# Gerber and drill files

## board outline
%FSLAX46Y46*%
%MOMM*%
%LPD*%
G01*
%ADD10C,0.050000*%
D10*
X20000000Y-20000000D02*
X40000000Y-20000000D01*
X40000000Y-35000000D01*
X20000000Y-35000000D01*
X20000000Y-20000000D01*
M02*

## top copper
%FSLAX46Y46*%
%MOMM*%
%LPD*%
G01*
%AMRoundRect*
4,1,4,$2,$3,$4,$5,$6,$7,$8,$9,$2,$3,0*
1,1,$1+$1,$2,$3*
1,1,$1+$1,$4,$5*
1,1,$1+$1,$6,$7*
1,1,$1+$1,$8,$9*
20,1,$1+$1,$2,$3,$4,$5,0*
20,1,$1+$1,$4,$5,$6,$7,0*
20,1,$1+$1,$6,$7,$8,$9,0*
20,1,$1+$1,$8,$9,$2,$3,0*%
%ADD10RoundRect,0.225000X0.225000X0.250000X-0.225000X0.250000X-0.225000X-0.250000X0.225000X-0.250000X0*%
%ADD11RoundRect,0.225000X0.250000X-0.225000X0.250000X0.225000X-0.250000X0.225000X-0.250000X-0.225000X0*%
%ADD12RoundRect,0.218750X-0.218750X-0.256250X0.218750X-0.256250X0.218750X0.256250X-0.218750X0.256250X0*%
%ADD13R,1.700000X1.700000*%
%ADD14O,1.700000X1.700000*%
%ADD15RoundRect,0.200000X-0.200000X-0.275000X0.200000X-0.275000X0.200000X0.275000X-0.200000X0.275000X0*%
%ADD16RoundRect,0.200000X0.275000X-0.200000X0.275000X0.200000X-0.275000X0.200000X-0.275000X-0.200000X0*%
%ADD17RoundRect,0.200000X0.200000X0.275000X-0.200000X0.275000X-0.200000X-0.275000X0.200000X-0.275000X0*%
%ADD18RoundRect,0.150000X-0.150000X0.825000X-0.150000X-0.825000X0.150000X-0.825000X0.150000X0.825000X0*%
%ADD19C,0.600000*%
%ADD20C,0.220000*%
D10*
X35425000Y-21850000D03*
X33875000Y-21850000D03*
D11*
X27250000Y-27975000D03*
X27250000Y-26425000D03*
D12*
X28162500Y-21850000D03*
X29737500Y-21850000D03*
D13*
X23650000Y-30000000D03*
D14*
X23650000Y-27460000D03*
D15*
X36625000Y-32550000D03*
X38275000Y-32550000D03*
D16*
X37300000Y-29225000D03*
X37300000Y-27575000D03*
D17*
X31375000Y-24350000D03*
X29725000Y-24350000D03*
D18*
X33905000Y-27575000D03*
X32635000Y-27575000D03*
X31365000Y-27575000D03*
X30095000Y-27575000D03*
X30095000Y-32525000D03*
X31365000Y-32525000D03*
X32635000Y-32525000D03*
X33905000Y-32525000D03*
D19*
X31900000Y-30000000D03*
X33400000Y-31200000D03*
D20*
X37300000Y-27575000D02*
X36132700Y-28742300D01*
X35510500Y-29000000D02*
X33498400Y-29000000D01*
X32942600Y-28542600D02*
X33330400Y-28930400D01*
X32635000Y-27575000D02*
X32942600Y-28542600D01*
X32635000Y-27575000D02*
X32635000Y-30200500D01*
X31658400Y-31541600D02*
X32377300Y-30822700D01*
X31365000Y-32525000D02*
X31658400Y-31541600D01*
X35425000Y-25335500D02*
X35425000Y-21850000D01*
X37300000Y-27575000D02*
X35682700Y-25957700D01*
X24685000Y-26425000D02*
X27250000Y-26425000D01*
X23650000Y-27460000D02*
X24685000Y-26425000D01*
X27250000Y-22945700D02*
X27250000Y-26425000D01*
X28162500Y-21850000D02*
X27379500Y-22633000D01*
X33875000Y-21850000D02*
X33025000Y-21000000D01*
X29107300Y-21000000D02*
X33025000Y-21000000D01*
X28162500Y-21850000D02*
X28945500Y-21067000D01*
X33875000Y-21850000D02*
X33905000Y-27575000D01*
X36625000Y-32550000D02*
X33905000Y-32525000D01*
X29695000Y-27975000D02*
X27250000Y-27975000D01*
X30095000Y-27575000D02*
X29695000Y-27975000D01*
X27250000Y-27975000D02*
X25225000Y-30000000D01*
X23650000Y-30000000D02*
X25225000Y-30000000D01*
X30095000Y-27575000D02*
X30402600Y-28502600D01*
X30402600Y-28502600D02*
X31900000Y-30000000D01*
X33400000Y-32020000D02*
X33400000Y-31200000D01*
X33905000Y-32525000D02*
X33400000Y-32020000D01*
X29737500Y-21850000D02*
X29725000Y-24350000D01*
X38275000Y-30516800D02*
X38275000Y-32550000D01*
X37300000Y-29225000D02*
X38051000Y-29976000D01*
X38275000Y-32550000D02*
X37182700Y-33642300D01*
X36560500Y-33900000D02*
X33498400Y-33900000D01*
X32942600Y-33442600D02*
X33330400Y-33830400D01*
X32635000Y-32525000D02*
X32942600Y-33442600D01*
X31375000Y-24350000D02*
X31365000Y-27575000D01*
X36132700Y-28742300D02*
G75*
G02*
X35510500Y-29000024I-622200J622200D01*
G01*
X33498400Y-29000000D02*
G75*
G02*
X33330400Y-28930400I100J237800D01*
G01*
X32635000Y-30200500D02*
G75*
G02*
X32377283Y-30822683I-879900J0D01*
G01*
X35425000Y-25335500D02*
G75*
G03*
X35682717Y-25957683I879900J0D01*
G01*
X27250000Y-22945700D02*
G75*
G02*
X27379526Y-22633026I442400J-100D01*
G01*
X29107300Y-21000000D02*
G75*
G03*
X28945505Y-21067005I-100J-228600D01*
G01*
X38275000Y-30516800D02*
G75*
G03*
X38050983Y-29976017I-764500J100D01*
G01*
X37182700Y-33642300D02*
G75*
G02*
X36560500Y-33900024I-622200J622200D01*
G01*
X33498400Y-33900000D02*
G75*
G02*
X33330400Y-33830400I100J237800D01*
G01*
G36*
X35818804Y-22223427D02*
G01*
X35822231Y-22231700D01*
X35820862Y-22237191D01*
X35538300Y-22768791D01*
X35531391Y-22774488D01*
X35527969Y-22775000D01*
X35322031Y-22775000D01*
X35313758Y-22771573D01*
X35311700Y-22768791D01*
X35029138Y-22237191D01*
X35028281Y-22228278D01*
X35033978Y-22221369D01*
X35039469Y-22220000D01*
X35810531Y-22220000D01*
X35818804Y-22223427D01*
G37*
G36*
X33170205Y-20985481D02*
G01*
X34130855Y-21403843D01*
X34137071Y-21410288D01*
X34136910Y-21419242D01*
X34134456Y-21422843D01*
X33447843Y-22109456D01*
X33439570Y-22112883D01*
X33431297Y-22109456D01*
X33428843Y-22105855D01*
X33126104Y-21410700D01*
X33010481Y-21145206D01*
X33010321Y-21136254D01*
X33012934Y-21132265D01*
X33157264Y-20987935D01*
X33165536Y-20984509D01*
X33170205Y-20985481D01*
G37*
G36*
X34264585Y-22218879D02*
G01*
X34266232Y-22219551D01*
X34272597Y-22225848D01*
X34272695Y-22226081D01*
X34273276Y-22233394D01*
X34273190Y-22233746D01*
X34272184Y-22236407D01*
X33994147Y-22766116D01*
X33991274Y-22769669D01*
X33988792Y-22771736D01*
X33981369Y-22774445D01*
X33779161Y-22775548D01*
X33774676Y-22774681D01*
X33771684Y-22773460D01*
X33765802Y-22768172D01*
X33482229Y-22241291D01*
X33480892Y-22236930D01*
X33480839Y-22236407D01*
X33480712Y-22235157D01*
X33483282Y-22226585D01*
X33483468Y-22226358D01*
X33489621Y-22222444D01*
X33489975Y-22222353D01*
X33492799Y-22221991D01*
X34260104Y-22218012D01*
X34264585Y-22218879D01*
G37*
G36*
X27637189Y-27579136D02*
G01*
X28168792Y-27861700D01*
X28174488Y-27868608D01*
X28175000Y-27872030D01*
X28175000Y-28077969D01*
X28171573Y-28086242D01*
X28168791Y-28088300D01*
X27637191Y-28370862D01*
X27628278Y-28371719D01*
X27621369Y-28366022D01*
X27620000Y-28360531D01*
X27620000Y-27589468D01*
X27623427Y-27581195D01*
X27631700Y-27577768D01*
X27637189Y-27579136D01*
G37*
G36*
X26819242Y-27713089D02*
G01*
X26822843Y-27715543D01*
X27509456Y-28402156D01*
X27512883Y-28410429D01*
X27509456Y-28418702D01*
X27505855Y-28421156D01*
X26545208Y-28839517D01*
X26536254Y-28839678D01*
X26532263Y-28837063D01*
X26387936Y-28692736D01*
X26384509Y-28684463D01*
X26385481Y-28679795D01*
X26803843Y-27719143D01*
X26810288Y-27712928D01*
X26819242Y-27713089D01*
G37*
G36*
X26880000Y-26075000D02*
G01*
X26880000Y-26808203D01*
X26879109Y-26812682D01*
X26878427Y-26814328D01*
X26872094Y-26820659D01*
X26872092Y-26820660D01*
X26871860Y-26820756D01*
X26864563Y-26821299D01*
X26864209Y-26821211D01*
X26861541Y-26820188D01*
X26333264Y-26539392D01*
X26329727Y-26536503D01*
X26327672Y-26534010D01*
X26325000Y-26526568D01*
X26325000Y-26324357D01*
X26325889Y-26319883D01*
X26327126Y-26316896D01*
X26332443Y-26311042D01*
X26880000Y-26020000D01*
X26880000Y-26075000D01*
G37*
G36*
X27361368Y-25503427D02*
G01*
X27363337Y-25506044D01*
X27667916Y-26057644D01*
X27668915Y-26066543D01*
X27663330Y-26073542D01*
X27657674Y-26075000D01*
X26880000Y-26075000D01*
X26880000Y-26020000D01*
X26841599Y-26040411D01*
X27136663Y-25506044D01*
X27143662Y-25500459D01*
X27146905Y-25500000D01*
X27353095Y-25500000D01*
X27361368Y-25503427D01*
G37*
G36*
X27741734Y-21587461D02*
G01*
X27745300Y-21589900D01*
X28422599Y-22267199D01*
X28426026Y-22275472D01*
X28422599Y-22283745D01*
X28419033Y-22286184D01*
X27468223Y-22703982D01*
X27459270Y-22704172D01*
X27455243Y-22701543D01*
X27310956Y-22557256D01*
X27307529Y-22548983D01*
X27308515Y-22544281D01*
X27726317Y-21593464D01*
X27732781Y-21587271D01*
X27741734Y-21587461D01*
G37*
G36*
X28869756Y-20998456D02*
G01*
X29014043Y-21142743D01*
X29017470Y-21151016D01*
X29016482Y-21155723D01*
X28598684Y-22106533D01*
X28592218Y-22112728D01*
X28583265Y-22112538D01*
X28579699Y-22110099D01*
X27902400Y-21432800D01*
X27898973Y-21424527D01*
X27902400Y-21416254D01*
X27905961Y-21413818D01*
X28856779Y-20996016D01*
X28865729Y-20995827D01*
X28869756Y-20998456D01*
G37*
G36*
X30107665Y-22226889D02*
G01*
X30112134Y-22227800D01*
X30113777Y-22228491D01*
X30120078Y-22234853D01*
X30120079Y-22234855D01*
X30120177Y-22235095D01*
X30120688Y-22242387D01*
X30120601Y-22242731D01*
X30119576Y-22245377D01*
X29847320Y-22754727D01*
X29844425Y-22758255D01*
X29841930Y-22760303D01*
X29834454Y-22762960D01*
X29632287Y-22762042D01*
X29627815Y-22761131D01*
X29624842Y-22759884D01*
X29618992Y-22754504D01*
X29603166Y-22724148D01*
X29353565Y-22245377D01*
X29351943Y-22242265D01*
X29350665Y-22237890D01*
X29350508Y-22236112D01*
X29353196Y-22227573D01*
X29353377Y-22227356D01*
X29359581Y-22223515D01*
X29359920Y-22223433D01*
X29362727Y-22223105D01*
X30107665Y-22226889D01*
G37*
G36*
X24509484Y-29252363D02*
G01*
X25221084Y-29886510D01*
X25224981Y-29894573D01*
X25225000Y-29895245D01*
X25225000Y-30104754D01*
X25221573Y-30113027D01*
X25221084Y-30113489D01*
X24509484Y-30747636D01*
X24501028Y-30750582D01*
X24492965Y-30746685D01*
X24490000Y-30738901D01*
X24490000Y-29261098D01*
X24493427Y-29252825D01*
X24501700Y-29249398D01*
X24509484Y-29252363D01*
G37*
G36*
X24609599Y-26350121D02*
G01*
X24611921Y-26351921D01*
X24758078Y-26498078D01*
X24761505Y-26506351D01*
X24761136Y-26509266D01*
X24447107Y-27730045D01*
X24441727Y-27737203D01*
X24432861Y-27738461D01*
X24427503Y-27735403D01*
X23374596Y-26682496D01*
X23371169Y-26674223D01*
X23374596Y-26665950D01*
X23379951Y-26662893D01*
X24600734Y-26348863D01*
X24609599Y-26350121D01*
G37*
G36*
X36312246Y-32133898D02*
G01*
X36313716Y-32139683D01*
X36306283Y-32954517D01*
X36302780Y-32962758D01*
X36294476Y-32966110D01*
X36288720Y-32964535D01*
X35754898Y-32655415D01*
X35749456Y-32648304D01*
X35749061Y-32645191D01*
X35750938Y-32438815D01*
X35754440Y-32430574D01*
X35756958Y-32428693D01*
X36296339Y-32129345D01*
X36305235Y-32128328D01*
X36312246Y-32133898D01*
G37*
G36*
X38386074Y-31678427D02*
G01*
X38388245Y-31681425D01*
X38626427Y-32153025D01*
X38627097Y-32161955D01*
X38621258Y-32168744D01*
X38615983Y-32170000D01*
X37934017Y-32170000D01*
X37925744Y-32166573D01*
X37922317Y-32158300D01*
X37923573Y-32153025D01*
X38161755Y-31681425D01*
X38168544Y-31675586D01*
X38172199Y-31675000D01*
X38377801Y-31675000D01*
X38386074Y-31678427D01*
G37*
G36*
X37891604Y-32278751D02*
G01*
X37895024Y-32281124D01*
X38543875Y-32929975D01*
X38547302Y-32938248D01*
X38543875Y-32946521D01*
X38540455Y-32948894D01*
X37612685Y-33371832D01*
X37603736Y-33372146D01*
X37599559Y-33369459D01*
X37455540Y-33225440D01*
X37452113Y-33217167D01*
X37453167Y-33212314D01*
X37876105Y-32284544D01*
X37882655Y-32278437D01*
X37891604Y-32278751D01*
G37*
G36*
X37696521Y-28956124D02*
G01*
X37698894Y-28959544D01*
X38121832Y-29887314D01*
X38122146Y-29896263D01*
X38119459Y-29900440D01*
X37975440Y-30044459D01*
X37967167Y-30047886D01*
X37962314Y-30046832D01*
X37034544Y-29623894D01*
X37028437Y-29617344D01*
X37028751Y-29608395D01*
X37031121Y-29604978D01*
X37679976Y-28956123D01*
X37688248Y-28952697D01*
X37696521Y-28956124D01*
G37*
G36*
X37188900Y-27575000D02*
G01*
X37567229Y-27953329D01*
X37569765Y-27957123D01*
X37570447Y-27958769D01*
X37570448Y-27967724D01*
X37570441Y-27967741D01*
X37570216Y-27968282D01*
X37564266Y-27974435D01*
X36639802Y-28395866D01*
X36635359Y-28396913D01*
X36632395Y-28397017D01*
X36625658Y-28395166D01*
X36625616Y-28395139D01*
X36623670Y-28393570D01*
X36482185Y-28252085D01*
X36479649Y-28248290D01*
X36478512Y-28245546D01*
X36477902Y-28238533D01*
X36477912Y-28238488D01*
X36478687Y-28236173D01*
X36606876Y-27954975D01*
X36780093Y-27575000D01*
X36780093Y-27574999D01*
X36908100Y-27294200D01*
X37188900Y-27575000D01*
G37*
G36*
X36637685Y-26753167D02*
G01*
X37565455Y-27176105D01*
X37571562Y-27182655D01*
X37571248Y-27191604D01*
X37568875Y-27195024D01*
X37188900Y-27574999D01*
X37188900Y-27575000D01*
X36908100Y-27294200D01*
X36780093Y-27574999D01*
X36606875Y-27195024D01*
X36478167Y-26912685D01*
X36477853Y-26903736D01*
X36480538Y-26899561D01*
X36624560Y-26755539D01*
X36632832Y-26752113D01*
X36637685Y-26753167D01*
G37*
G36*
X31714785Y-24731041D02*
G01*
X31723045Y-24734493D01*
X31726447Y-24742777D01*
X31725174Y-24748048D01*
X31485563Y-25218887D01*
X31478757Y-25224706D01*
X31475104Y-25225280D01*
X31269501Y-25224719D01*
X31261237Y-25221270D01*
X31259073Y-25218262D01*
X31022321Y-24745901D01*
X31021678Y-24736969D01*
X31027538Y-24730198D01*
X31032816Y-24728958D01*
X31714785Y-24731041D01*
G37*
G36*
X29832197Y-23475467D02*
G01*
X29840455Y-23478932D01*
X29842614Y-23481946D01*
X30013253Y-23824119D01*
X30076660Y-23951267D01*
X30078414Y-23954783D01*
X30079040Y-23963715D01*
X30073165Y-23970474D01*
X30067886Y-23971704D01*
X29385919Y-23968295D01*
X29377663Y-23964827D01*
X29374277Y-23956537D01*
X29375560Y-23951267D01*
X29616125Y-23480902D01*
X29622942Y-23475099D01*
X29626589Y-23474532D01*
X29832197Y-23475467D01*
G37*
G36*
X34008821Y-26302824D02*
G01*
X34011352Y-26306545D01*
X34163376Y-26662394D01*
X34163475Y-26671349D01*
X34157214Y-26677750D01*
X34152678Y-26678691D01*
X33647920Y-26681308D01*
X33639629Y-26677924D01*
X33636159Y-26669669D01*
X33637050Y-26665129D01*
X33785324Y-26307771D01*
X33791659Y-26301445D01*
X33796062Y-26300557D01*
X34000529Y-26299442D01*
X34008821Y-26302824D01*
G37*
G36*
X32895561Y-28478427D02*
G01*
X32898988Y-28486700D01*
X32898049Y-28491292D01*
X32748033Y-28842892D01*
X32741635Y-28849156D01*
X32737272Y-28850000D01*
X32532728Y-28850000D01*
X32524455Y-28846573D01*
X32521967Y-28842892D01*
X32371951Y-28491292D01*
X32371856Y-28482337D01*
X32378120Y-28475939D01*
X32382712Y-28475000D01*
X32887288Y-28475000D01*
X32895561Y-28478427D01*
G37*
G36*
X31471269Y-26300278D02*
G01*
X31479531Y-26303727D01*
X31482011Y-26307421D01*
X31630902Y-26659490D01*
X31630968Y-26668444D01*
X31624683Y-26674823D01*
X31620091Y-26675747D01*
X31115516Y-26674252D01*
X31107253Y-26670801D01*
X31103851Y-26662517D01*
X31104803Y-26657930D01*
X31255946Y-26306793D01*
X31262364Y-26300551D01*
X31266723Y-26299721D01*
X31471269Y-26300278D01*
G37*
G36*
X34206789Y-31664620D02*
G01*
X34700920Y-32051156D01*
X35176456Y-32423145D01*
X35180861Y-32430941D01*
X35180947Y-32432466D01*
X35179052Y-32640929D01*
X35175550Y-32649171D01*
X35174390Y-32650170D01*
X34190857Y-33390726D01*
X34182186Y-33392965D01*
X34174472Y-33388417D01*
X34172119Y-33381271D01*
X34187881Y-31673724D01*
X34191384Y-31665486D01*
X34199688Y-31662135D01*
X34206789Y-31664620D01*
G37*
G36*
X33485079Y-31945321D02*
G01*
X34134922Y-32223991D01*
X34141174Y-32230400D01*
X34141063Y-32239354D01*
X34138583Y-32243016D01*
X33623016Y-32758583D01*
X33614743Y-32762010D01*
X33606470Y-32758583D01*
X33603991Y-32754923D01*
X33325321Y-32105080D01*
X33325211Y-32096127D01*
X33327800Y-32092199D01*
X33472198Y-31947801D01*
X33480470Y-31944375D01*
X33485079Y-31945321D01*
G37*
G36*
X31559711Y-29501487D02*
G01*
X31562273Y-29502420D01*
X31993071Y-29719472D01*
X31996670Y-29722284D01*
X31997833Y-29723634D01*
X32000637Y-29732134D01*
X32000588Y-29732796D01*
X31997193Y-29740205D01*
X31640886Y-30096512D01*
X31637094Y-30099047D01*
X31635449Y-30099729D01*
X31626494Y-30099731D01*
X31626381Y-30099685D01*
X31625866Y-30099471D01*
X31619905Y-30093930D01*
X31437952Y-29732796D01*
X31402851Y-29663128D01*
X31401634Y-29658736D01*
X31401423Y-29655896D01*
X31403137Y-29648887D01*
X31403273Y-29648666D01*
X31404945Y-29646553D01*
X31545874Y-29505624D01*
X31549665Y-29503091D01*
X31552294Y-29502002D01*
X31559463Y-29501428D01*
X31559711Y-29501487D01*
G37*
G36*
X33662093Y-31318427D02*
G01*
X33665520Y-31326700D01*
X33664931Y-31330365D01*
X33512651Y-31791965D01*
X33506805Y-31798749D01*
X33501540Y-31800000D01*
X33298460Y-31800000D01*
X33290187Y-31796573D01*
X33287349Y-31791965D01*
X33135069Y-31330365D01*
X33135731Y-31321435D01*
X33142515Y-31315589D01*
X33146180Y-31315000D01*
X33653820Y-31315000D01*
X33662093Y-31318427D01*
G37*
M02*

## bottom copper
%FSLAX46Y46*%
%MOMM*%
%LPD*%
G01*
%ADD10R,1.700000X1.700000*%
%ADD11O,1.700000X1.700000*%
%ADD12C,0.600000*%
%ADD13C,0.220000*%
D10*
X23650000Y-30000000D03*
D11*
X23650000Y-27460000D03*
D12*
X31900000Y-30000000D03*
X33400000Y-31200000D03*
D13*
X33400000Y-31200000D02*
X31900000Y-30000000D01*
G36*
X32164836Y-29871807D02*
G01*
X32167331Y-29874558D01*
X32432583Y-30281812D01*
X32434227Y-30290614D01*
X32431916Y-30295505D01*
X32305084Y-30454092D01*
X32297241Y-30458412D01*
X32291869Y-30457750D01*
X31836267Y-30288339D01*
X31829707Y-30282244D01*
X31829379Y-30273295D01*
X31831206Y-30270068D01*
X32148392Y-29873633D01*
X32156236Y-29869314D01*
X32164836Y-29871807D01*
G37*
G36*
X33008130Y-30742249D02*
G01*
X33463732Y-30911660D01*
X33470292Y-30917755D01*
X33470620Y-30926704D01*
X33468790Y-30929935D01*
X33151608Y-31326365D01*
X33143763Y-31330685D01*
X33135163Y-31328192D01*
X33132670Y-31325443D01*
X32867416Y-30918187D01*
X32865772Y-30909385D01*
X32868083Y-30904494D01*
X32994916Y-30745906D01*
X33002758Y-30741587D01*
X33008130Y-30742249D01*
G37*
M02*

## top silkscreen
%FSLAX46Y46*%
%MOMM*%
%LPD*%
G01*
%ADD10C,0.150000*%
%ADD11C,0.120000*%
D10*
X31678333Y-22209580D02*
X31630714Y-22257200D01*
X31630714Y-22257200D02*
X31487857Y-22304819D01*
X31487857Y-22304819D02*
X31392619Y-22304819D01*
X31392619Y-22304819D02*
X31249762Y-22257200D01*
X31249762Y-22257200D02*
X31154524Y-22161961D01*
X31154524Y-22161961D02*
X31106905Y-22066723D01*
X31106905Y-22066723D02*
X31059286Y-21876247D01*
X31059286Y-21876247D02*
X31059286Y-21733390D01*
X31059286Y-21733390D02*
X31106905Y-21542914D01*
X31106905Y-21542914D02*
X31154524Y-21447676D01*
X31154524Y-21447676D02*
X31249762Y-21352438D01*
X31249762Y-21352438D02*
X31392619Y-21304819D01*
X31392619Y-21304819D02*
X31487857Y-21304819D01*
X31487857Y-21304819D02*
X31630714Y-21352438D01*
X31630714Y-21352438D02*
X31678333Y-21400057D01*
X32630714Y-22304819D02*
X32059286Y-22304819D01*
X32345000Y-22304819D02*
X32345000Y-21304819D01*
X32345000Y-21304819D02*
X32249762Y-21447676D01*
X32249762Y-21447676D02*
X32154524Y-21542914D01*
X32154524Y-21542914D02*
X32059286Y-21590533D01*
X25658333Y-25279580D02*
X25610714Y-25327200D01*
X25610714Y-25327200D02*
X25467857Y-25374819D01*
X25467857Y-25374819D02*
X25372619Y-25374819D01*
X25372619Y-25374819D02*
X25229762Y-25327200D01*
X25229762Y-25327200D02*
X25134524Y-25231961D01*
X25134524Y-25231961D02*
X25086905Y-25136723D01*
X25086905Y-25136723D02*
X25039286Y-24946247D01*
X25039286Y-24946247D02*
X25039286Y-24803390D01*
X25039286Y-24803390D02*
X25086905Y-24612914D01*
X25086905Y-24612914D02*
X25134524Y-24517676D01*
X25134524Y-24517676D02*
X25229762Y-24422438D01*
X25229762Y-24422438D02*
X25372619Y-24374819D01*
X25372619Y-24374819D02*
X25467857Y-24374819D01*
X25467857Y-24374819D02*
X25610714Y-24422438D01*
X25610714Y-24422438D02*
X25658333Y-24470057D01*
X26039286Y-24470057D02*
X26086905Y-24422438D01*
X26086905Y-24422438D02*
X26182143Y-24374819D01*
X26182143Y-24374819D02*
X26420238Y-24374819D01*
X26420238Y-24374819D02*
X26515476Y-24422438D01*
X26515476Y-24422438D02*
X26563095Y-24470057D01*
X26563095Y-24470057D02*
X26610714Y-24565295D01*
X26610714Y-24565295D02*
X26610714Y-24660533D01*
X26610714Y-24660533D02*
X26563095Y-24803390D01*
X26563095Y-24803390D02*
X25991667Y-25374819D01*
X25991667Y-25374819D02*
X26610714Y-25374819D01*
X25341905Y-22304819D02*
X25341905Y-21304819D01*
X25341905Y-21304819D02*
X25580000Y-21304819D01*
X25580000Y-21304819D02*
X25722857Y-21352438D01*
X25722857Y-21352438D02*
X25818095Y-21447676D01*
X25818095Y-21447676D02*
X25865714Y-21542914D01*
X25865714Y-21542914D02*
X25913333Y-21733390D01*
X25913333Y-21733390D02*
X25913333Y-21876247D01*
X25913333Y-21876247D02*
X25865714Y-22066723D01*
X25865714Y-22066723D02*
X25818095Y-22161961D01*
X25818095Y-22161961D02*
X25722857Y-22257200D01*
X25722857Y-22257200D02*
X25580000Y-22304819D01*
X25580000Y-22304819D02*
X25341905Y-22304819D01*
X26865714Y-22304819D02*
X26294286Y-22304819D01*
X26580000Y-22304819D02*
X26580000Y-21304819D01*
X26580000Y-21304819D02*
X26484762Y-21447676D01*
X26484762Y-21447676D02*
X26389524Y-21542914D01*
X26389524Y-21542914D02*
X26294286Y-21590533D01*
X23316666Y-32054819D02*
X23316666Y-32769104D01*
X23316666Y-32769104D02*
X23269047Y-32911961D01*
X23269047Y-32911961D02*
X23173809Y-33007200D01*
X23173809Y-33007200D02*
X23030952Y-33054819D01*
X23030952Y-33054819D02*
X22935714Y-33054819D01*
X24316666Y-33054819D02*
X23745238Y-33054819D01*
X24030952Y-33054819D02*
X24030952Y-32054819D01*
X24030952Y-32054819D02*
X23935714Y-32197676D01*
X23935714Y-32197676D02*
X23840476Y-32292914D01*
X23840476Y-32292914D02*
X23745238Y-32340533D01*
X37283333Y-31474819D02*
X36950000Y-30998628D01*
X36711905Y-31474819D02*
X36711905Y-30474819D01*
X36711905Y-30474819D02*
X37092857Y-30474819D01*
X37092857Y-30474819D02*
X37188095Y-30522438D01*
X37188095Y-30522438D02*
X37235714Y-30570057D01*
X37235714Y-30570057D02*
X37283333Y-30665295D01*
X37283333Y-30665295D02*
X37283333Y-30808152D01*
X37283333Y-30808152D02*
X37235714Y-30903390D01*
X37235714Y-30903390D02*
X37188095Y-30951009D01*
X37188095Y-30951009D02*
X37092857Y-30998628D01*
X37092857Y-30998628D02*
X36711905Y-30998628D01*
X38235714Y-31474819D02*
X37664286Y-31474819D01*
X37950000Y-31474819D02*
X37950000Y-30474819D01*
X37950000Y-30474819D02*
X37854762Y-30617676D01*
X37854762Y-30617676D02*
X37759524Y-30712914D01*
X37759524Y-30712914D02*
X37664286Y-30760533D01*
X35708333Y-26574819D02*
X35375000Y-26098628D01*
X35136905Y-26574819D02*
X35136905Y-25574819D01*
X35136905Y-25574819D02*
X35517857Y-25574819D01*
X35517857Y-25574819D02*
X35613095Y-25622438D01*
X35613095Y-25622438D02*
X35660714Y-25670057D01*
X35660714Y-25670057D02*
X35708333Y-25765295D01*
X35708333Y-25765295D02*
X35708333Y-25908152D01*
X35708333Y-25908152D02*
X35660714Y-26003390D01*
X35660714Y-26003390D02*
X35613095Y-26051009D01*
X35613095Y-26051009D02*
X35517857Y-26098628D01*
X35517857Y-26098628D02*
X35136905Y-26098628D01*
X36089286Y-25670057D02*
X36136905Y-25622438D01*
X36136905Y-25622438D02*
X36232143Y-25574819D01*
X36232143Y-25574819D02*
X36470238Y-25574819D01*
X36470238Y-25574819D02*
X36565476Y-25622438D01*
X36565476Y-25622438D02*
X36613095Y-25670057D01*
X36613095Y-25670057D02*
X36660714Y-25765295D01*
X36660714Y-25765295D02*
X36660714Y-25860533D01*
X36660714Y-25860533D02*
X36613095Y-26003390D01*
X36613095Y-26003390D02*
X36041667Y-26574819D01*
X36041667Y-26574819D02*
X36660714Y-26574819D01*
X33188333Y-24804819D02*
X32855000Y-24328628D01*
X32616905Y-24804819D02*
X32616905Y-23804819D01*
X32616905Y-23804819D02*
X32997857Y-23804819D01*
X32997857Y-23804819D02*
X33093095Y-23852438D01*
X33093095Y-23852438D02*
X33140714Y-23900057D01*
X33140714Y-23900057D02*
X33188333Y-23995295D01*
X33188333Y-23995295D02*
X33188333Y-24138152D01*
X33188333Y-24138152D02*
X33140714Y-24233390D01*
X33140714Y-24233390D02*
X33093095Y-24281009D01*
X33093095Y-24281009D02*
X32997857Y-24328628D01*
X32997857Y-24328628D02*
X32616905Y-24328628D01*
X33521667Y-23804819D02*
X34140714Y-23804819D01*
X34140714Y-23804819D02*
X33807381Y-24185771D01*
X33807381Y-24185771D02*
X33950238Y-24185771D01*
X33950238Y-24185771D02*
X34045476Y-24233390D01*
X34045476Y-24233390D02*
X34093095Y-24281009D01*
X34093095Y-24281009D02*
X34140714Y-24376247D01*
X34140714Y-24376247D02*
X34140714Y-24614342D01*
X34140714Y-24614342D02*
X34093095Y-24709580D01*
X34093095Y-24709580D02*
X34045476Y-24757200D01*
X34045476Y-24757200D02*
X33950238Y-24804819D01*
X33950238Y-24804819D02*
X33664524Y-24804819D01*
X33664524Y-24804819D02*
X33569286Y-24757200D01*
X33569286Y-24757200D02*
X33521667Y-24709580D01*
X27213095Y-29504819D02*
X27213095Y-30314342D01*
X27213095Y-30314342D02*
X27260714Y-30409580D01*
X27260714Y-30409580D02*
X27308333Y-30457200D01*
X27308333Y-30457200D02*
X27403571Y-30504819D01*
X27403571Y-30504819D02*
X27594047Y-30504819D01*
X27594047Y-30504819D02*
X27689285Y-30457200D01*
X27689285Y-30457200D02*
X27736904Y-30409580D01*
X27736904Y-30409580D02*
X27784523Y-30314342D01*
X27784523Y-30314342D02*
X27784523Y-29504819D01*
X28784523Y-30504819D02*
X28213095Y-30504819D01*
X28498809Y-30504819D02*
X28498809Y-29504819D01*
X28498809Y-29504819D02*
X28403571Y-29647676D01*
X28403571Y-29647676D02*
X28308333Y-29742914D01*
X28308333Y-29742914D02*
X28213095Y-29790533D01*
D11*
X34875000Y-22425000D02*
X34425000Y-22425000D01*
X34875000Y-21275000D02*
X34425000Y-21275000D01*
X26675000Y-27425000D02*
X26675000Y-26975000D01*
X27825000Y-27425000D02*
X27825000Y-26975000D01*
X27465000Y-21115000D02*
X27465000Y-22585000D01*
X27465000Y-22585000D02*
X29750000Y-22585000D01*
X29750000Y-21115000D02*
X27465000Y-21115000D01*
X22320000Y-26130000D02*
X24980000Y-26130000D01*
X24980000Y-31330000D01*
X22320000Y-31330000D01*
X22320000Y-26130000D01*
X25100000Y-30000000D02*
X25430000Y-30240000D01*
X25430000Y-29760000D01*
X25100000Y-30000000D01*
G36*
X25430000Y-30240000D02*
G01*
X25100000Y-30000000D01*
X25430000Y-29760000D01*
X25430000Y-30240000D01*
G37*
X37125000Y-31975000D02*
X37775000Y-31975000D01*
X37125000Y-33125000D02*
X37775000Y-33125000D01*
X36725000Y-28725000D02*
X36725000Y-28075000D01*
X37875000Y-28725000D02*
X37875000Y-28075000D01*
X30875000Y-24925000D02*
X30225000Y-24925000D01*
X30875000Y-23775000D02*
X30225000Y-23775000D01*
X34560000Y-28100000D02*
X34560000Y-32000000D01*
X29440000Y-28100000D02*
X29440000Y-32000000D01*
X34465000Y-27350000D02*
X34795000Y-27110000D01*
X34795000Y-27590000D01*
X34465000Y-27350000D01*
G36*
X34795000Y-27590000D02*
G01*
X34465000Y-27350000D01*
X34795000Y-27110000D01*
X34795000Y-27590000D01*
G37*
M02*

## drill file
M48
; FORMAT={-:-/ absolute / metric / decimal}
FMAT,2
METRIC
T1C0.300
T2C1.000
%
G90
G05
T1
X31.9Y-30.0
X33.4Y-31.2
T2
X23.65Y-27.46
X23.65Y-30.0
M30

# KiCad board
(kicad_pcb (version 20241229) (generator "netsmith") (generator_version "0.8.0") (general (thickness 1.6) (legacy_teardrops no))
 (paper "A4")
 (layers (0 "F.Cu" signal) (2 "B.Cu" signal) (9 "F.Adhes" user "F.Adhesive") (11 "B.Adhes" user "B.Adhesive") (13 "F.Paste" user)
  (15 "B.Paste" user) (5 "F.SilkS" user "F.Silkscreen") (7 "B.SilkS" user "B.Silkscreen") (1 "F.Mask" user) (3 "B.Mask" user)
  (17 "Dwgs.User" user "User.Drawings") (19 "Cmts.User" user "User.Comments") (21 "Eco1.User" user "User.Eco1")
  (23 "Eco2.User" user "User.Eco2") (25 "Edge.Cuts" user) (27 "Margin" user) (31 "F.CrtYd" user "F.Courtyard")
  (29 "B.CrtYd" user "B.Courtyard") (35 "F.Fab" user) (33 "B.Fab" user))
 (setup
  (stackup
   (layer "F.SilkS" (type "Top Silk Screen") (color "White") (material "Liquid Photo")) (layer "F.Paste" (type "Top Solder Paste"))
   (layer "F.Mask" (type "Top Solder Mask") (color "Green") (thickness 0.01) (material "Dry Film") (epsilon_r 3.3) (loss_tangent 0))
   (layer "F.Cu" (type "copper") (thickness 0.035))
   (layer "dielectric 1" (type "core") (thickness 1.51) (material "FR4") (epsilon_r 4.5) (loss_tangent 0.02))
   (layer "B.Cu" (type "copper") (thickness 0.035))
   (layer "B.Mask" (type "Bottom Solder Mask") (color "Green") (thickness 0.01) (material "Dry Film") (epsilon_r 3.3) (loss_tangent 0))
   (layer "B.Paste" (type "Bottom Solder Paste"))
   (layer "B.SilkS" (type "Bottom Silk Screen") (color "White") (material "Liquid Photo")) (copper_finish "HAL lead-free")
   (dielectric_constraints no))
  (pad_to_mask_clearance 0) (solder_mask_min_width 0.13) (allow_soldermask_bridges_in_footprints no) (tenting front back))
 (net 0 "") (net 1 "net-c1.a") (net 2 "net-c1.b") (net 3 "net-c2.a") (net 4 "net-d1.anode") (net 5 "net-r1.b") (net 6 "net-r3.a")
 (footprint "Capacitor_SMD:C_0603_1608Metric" (layer "F.Cu") (at 34.65 21.85 180)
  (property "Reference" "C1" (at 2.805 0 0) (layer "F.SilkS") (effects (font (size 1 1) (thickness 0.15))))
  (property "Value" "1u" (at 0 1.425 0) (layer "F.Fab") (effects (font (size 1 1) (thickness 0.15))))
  (pad "1" smd roundrect (at -0.775 0 180) (size 0.9 0.95) (layers "F.Cu" "F.Mask" "F.Paste") (roundrect_rratio 0.25) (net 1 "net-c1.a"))
  (pad "2" smd roundrect (at 0.775 0 180) (size 0.9 0.95) (layers "F.Cu" "F.Mask" "F.Paste") (roundrect_rratio 0.25) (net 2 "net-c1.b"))
  (fp_line (start -0.225 -0.575) (end 0.225 -0.575) (stroke (width 0.12) (type solid)) (layer "F.SilkS"))
  (fp_line (start -0.225 0.575) (end 0.225 0.575) (stroke (width 0.12) (type solid)) (layer "F.SilkS")))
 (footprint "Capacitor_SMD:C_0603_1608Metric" (layer "F.Cu") (at 27.25 27.2 90)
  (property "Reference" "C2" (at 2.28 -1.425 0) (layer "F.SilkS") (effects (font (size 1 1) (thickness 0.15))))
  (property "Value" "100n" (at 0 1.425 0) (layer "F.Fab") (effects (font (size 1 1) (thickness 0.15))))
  (pad "1" smd roundrect (at -0.775 0 90) (size 0.9 0.95) (layers "F.Cu" "F.Mask" "F.Paste") (roundrect_rratio 0.25) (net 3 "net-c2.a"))
  (pad "2" smd roundrect (at 0.775 0 90) (size 0.9 0.95) (layers "F.Cu" "F.Mask" "F.Paste") (roundrect_rratio 0.25) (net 2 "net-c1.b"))
  (fp_line (start -0.225 -0.575) (end 0.225 -0.575) (stroke (width 0.12) (type solid)) (layer "F.SilkS"))
  (fp_line (start -0.225 0.575) (end 0.225 0.575) (stroke (width 0.12) (type solid)) (layer "F.SilkS")))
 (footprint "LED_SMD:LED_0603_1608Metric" (layer "F.Cu") (at 28.95 21.85)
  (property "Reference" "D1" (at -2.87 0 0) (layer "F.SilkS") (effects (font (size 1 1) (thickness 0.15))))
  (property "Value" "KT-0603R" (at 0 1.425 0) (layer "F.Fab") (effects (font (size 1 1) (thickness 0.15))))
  (pad "1" smd roundrect (at -0.7875 0) (size 0.875 0.95) (layers "F.Cu" "F.Mask" "F.Paste") (roundrect_rratio 0.25) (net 2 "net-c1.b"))
  (pad "2" smd roundrect (at 0.7875 0) (size 0.875 0.95) (layers "F.Cu" "F.Mask" "F.Paste") (roundrect_rratio 0.25) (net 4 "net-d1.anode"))
  (fp_line (start -1.485 -0.735) (end -1.485 0.735) (stroke (width 0.12) (type solid)) (layer "F.SilkS"))
  (fp_line (start -1.485 0.735) (end 0.8 0.735) (stroke (width 0.12) (type solid)) (layer "F.SilkS"))
  (fp_line (start 0.8 -0.735) (end -1.485 -0.735) (stroke (width 0.12) (type solid)) (layer "F.SilkS")))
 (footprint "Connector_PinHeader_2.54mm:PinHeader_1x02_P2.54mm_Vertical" (layer "F.Cu") (at 23.65 30 180)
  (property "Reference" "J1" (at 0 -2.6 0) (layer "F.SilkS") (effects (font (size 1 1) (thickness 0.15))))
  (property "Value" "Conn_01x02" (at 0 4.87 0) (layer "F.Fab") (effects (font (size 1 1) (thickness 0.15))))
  (pad "1" thru_hole rect (at 0 0 180) (size 1.7 1.7) (drill 1) (layers "*.Cu" "*.Mask") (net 3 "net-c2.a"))
  (pad "2" thru_hole oval (at 0 2.54 180) (size 1.7 1.7) (drill 1) (layers "*.Cu" "*.Mask") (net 2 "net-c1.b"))
  (fp_rect (start -1.33 -1.33) (end 1.33 3.87) (stroke (width 0.12) (type solid)) (fill no) (layer "F.SilkS"))
  (fp_poly (pts (xy -1.45 0) (xy -1.78 -0.24) (xy -1.78 0.24)) (stroke (width 0.12) (type solid)) (fill solid) (layer "F.SilkS")))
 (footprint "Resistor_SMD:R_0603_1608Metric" (layer "F.Cu") (at 37.45 32.55)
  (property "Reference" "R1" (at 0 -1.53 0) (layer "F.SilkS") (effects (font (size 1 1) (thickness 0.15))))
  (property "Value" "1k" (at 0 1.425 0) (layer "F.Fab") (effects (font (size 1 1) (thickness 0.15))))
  (pad "1" smd roundrect (at -0.825 0) (size 0.8 0.95) (layers "F.Cu" "F.Mask" "F.Paste") (roundrect_rratio 0.25) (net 3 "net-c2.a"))
  (pad "2" smd roundrect (at 0.825 0) (size 0.8 0.95) (layers "F.Cu" "F.Mask" "F.Paste") (roundrect_rratio 0.25) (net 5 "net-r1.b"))
  (fp_line (start -0.325 -0.575) (end 0.325 -0.575) (stroke (width 0.12) (type solid)) (layer "F.SilkS"))
  (fp_line (start -0.325 0.575) (end 0.325 0.575) (stroke (width 0.12) (type solid)) (layer "F.SilkS")))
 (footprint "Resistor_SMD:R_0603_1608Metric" (layer "F.Cu") (at 37.3 28.4 90)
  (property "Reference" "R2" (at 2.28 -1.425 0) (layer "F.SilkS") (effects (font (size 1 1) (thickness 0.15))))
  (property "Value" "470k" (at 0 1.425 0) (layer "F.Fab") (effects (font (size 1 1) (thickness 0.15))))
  (pad "1" smd roundrect (at -0.825 0 90) (size 0.8 0.95) (layers "F.Cu" "F.Mask" "F.Paste") (roundrect_rratio 0.25) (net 5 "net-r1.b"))
  (pad "2" smd roundrect (at 0.825 0 90) (size 0.8 0.95) (layers "F.Cu" "F.Mask" "F.Paste") (roundrect_rratio 0.25) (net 1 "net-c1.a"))
  (fp_line (start -0.325 -0.575) (end 0.325 -0.575) (stroke (width 0.12) (type solid)) (layer "F.SilkS"))
  (fp_line (start -0.325 0.575) (end 0.325 0.575) (stroke (width 0.12) (type solid)) (layer "F.SilkS")))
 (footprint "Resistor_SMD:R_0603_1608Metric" (layer "F.Cu") (at 30.55 24.35 180)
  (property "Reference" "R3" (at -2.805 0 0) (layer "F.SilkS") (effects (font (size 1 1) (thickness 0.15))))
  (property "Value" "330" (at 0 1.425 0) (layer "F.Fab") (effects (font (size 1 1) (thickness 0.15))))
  (pad "1" smd roundrect (at -0.825 0 180) (size 0.8 0.95) (layers "F.Cu" "F.Mask" "F.Paste") (roundrect_rratio 0.25) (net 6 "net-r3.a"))
  (pad "2" smd roundrect (at 0.825 0 180) (size 0.8 0.95) (layers "F.Cu" "F.Mask" "F.Paste") (roundrect_rratio 0.25) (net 4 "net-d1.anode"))
  (fp_line (start -0.325 -0.575) (end 0.325 -0.575) (stroke (width 0.12) (type solid)) (layer "F.SilkS"))
  (fp_line (start -0.325 0.575) (end 0.325 0.575) (stroke (width 0.12) (type solid)) (layer "F.SilkS")))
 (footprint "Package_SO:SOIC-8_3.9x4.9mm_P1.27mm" (layer "F.Cu") (at 32 30.05 270)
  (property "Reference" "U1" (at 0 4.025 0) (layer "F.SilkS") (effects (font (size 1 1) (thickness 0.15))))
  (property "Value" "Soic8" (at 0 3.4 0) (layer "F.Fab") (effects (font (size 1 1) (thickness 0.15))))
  (pad "1" smd roundrect (at -2.475 -1.905 270) (size 1.95 0.6) (layers "F.Cu" "F.Mask" "F.Paste") (roundrect_rratio 0.25)
   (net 2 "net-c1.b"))
  (pad "2" smd roundrect (at -2.475 -0.635 270) (size 1.95 0.6) (layers "F.Cu" "F.Mask" "F.Paste") (roundrect_rratio 0.25)
   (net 1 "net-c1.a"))
  (pad "3" smd roundrect (at -2.475 0.635 270) (size 1.95 0.6) (layers "F.Cu" "F.Mask" "F.Paste") (roundrect_rratio 0.25) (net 6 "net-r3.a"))
  (pad "4" smd roundrect (at -2.475 1.905 270) (size 1.95 0.6) (layers "F.Cu" "F.Mask" "F.Paste") (roundrect_rratio 0.25) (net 3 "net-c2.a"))
  (pad "5" smd roundrect (at 2.475 1.905 270) (size 1.95 0.6) (layers "F.Cu" "F.Mask" "F.Paste") (roundrect_rratio 0.25))
  (pad "6" smd roundrect (at 2.475 0.635 270) (size 1.95 0.6) (layers "F.Cu" "F.Mask" "F.Paste") (roundrect_rratio 0.25) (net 1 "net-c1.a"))
  (pad "7" smd roundrect (at 2.475 -0.635 270) (size 1.95 0.6) (layers "F.Cu" "F.Mask" "F.Paste") (roundrect_rratio 0.25) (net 5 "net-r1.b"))
  (pad "8" smd roundrect (at 2.475 -1.905 270) (size 1.95 0.6) (layers "F.Cu" "F.Mask" "F.Paste") (roundrect_rratio 0.25) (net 3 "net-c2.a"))
  (fp_line (start -1.95 -2.56) (end 1.95 -2.56) (stroke (width 0.12) (type solid)) (layer "F.SilkS"))
  (fp_line (start -1.95 2.56) (end 1.95 2.56) (stroke (width 0.12) (type solid)) (layer "F.SilkS"))
  (fp_poly (pts (xy -2.7 -2.465) (xy -2.94 -2.795) (xy -2.46 -2.795)) (stroke (width 0.12) (type solid)) (fill solid) (layer "F.SilkS")))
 (segment (start 37.3 27.575) (end 36.1327 28.7423) (width 0.22) (layer "F.Cu") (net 1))
 (segment (start 35.5105 29) (end 33.4984 29) (width 0.22) (layer "F.Cu") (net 1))
 (segment (start 32.9426 28.5426) (end 33.3304 28.9304) (width 0.22) (layer "F.Cu") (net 1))
 (segment (start 32.635 27.575) (end 32.9426 28.5426) (width 0.22) (layer "F.Cu") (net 1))
 (segment (start 32.635 27.575) (end 32.635 30.2005) (width 0.22) (layer "F.Cu") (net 1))
 (segment (start 31.6584 31.5416) (end 32.3773 30.8227) (width 0.22) (layer "F.Cu") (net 1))
 (segment (start 31.365 32.525) (end 31.6584 31.5416) (width 0.22) (layer "F.Cu") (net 1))
 (segment (start 35.425 25.3355) (end 35.425 21.85) (width 0.22) (layer "F.Cu") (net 1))
 (segment (start 37.3 27.575) (end 35.6827 25.9577) (width 0.22) (layer "F.Cu") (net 1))
 (segment (start 24.685 26.425) (end 27.25 26.425) (width 0.22) (layer "F.Cu") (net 2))
 (segment (start 23.65 27.46) (end 24.685 26.425) (width 0.22) (layer "F.Cu") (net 2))
 (segment (start 27.25 22.9457) (end 27.25 26.425) (width 0.22) (layer "F.Cu") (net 2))
 (segment (start 28.1625 21.85) (end 27.3795 22.633) (width 0.22) (layer "F.Cu") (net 2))
 (segment (start 33.875 21.85) (end 33.025 21) (width 0.22) (layer "F.Cu") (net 2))
 (segment (start 29.1073 21) (end 33.025 21) (width 0.22) (layer "F.Cu") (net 2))
 (segment (start 28.1625 21.85) (end 28.9455 21.067) (width 0.22) (layer "F.Cu") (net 2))
 (segment (start 33.875 21.85) (end 33.905 27.575) (width 0.22) (layer "F.Cu") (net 2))
 (segment (start 36.625 32.55) (end 33.905 32.525) (width 0.22) (layer "F.Cu") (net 3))
 (segment (start 29.695 27.975) (end 27.25 27.975) (width 0.22) (layer "F.Cu") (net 3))
 (segment (start 30.095 27.575) (end 29.695 27.975) (width 0.22) (layer "F.Cu") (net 3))
 (segment (start 27.25 27.975) (end 25.225 30) (width 0.22) (layer "F.Cu") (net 3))
 (segment (start 23.65 30) (end 25.225 30) (width 0.22) (layer "F.Cu") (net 3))
 (segment (start 30.095 27.575) (end 30.4026 28.5026) (width 0.22) (layer "F.Cu") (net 3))
 (segment (start 30.4026 28.5026) (end 31.9 30) (width 0.22) (layer "F.Cu") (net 3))
 (segment (start 33.4 31.2) (end 31.9 30) (width 0.22) (layer "B.Cu") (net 3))
 (segment (start 33.4 32.02) (end 33.4 31.2) (width 0.22) (layer "F.Cu") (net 3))
 (segment (start 33.905 32.525) (end 33.4 32.02) (width 0.22) (layer "F.Cu") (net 3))
 (segment (start 29.7375 21.85) (end 29.725 24.35) (width 0.22) (layer "F.Cu") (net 4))
 (segment (start 38.275 30.5168) (end 38.275 32.55) (width 0.22) (layer "F.Cu") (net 5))
 (segment (start 37.3 29.225) (end 38.051 29.976) (width 0.22) (layer "F.Cu") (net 5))
 (segment (start 38.275 32.55) (end 37.1827 33.6423) (width 0.22) (layer "F.Cu") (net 5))
 (segment (start 36.5605 33.9) (end 33.4984 33.9) (width 0.22) (layer "F.Cu") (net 5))
 (segment (start 32.9426 33.4426) (end 33.3304 33.8304) (width 0.22) (layer "F.Cu") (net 5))
 (segment (start 32.635 32.525) (end 32.9426 33.4426) (width 0.22) (layer "F.Cu") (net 5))
 (segment (start 31.375 24.35) (end 31.365 27.575) (width 0.22) (layer "F.Cu") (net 6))
 (arc (start 36.1327 28.7423) (mid 35.8473 28.933) (end 35.5105 29) (width 0.22) (layer "F.Cu") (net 1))
 (arc (start 33.4984 29) (mid 33.4075 28.9819) (end 33.3304 28.9304) (width 0.22) (layer "F.Cu") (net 1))
 (arc (start 32.635 30.2005) (mid 32.568 30.5373) (end 32.3773 30.8227) (width 0.22) (layer "F.Cu") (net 1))
 (arc (start 35.425 25.3355) (mid 35.492 25.6723) (end 35.6827 25.9577) (width 0.22) (layer "F.Cu") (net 1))
 (arc (start 27.25 22.9457) (mid 27.2837 22.7764) (end 27.3795 22.633) (width 0.22) (layer "F.Cu") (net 2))
 (arc (start 29.1073 21) (mid 29.0197 21.0174) (end 28.9455 21.067) (width 0.22) (layer "F.Cu") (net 2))
 (arc (start 38.275 30.5168) (mid 38.2168 30.2241) (end 38.051 29.976) (width 0.22) (layer "F.Cu") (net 5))
 (arc (start 37.1827 33.6423) (mid 36.8973 33.833) (end 36.5605 33.9) (width 0.22) (layer "F.Cu") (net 5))
 (arc (start 33.4984 33.9) (mid 33.4075 33.8819) (end 33.3304 33.8304) (width 0.22) (layer "F.Cu") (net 5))
 (via (at 31.9 30) (size 0.6) (drill 0.3) (layers "F.Cu" "B.Cu") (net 3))
 (via (at 33.4 31.2) (size 0.6) (drill 0.3) (layers "F.Cu" "B.Cu") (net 3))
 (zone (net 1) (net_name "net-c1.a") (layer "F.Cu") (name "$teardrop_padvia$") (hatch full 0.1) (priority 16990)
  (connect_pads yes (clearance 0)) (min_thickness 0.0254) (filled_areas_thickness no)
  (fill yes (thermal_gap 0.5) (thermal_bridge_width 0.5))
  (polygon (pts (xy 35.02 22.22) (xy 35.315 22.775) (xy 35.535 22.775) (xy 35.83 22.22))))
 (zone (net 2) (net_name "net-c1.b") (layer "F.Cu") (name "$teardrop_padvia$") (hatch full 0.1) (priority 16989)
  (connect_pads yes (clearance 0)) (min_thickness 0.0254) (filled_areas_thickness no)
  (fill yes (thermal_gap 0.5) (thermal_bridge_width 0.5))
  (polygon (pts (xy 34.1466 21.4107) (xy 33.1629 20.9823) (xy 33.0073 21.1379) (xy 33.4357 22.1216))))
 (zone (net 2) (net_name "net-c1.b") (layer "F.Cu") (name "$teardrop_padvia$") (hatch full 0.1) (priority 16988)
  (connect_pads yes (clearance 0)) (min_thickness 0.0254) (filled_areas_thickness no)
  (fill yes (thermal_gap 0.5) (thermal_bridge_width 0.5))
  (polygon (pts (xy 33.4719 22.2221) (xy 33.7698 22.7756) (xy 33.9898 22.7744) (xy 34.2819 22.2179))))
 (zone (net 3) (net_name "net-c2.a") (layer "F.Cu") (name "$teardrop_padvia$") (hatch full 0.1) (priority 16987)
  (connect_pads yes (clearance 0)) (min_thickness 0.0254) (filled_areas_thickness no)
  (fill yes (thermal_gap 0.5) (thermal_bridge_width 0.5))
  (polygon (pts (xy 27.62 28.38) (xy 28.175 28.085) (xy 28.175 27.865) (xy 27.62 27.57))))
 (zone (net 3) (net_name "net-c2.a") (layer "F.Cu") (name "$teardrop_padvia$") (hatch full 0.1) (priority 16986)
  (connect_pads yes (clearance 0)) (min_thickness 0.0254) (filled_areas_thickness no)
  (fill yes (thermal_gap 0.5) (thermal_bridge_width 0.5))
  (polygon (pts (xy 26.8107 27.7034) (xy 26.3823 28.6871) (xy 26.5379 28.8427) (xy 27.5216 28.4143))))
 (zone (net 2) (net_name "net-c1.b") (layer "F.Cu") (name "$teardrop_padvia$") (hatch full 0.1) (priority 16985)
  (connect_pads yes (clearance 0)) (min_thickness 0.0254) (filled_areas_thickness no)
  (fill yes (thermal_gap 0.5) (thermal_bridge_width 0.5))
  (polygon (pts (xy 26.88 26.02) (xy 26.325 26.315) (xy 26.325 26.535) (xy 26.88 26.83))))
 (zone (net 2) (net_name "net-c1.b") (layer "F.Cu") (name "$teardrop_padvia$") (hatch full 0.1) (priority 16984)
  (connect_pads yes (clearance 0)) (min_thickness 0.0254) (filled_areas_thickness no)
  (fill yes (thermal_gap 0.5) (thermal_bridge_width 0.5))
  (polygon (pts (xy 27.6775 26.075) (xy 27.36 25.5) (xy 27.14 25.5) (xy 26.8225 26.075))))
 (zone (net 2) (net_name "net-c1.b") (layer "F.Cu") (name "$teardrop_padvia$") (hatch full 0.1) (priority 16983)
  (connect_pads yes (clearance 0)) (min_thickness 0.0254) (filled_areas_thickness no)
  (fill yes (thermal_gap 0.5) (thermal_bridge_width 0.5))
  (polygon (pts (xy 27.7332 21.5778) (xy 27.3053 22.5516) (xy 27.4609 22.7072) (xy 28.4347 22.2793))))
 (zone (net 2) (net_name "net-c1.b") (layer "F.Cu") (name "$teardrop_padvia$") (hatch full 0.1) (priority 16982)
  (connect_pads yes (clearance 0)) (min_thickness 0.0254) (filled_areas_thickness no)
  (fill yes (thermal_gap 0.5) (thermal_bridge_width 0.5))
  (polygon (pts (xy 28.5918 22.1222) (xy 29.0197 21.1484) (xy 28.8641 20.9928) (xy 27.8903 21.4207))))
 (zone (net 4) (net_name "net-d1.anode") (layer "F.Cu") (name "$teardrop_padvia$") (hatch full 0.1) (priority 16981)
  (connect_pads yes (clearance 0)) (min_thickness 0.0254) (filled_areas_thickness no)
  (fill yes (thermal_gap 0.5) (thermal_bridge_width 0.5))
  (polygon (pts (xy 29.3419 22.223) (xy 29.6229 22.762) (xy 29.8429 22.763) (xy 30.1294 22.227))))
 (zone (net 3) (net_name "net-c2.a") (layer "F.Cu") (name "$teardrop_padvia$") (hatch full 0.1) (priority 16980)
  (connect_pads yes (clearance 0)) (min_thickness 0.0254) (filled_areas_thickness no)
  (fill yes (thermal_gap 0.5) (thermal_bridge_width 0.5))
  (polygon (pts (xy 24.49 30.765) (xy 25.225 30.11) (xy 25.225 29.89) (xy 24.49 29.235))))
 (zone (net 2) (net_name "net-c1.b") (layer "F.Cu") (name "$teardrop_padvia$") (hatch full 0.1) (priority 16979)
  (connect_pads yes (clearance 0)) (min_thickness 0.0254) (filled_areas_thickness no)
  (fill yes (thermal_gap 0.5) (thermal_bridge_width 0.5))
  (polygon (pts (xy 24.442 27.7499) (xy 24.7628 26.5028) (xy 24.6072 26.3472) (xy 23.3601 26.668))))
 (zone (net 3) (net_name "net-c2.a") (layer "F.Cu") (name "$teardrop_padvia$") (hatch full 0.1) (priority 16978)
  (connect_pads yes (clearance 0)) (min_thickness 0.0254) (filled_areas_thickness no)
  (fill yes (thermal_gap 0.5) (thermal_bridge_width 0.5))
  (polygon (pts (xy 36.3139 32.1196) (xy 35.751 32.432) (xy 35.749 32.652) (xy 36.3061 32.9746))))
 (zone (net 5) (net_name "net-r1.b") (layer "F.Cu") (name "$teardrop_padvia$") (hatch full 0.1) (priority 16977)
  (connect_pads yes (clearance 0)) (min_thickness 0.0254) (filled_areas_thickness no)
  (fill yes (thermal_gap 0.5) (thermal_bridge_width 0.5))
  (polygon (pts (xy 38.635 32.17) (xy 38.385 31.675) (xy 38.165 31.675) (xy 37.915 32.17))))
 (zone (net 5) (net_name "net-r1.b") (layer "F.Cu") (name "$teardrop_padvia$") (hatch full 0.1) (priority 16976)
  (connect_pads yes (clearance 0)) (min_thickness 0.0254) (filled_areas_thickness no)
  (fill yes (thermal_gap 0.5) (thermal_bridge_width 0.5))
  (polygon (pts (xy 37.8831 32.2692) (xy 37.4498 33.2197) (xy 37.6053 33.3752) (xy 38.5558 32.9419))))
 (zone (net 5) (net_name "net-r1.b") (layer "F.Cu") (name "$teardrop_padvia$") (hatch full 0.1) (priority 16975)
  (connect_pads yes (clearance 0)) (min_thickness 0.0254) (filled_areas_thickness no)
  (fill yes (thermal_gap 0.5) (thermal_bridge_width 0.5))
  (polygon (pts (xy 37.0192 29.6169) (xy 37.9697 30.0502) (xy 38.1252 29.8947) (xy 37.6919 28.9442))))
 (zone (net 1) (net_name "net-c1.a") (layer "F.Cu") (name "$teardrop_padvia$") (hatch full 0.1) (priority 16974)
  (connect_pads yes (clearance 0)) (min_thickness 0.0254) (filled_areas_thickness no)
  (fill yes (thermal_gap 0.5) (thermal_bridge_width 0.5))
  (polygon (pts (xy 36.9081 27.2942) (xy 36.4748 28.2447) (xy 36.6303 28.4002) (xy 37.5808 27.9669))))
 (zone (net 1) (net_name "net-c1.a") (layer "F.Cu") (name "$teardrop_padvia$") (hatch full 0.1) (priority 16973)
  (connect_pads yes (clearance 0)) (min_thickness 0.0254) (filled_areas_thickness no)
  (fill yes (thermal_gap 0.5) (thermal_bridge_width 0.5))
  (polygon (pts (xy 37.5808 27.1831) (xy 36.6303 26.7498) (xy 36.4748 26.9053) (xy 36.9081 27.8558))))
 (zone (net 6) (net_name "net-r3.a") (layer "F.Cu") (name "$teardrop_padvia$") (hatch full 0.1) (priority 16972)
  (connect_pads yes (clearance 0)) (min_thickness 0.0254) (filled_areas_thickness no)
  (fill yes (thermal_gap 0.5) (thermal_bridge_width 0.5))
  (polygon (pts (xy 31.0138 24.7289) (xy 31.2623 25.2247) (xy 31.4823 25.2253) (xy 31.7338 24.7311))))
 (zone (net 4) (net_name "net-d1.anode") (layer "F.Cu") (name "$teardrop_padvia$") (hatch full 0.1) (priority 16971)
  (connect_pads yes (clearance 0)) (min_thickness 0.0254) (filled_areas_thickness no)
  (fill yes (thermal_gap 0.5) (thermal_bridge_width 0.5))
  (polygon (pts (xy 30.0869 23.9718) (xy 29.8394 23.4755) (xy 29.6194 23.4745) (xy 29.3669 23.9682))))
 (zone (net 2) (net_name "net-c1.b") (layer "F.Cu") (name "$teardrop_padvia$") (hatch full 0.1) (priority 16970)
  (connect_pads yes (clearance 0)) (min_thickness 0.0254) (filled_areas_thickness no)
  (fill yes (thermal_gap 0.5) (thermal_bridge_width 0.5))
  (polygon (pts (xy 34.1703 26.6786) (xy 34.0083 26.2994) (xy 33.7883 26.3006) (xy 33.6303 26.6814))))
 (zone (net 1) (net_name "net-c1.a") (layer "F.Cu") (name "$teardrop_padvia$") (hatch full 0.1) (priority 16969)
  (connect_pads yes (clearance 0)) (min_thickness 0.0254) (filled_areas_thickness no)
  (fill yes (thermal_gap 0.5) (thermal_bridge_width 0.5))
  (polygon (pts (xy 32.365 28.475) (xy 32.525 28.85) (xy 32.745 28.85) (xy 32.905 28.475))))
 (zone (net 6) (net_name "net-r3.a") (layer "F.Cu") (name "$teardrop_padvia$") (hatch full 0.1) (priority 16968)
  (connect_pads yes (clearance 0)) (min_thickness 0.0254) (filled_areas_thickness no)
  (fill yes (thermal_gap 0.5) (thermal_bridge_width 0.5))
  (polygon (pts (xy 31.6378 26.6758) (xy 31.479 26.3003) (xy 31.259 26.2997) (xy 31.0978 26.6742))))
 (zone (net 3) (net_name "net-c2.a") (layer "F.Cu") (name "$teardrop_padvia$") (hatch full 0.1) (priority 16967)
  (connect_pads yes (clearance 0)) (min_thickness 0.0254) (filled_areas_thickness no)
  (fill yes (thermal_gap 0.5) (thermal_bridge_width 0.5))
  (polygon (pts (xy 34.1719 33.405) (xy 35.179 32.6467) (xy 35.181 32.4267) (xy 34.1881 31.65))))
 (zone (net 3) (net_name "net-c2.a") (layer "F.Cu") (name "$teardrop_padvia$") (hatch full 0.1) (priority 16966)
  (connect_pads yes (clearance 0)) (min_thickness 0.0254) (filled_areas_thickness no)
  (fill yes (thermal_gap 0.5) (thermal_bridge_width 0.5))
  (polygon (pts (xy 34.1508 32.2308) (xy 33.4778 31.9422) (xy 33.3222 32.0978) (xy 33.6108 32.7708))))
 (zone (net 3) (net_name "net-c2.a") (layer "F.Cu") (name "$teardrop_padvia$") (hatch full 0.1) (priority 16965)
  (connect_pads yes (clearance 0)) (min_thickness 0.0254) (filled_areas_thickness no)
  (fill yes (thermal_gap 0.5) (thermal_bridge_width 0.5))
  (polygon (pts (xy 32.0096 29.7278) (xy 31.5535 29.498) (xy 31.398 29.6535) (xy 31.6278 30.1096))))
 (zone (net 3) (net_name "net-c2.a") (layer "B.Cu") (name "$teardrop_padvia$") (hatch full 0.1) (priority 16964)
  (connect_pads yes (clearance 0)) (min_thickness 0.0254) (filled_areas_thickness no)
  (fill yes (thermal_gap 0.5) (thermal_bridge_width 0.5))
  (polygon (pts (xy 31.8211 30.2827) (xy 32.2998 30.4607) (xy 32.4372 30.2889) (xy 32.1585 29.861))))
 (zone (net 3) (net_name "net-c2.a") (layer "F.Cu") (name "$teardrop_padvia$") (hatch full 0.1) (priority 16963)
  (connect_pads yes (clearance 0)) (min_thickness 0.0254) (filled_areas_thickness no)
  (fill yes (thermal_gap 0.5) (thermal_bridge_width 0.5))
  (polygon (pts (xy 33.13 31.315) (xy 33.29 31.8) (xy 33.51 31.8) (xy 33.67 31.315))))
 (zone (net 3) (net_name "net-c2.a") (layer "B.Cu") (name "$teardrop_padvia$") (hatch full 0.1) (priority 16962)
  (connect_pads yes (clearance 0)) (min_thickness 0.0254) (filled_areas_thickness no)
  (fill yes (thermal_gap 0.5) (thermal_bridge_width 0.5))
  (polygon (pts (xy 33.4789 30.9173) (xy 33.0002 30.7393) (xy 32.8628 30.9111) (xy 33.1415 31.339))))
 (gr_rect (start 20 20) (end 40 35) (stroke (width 0.05) (type default)) (fill no) (layer "Edge.Cuts")))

